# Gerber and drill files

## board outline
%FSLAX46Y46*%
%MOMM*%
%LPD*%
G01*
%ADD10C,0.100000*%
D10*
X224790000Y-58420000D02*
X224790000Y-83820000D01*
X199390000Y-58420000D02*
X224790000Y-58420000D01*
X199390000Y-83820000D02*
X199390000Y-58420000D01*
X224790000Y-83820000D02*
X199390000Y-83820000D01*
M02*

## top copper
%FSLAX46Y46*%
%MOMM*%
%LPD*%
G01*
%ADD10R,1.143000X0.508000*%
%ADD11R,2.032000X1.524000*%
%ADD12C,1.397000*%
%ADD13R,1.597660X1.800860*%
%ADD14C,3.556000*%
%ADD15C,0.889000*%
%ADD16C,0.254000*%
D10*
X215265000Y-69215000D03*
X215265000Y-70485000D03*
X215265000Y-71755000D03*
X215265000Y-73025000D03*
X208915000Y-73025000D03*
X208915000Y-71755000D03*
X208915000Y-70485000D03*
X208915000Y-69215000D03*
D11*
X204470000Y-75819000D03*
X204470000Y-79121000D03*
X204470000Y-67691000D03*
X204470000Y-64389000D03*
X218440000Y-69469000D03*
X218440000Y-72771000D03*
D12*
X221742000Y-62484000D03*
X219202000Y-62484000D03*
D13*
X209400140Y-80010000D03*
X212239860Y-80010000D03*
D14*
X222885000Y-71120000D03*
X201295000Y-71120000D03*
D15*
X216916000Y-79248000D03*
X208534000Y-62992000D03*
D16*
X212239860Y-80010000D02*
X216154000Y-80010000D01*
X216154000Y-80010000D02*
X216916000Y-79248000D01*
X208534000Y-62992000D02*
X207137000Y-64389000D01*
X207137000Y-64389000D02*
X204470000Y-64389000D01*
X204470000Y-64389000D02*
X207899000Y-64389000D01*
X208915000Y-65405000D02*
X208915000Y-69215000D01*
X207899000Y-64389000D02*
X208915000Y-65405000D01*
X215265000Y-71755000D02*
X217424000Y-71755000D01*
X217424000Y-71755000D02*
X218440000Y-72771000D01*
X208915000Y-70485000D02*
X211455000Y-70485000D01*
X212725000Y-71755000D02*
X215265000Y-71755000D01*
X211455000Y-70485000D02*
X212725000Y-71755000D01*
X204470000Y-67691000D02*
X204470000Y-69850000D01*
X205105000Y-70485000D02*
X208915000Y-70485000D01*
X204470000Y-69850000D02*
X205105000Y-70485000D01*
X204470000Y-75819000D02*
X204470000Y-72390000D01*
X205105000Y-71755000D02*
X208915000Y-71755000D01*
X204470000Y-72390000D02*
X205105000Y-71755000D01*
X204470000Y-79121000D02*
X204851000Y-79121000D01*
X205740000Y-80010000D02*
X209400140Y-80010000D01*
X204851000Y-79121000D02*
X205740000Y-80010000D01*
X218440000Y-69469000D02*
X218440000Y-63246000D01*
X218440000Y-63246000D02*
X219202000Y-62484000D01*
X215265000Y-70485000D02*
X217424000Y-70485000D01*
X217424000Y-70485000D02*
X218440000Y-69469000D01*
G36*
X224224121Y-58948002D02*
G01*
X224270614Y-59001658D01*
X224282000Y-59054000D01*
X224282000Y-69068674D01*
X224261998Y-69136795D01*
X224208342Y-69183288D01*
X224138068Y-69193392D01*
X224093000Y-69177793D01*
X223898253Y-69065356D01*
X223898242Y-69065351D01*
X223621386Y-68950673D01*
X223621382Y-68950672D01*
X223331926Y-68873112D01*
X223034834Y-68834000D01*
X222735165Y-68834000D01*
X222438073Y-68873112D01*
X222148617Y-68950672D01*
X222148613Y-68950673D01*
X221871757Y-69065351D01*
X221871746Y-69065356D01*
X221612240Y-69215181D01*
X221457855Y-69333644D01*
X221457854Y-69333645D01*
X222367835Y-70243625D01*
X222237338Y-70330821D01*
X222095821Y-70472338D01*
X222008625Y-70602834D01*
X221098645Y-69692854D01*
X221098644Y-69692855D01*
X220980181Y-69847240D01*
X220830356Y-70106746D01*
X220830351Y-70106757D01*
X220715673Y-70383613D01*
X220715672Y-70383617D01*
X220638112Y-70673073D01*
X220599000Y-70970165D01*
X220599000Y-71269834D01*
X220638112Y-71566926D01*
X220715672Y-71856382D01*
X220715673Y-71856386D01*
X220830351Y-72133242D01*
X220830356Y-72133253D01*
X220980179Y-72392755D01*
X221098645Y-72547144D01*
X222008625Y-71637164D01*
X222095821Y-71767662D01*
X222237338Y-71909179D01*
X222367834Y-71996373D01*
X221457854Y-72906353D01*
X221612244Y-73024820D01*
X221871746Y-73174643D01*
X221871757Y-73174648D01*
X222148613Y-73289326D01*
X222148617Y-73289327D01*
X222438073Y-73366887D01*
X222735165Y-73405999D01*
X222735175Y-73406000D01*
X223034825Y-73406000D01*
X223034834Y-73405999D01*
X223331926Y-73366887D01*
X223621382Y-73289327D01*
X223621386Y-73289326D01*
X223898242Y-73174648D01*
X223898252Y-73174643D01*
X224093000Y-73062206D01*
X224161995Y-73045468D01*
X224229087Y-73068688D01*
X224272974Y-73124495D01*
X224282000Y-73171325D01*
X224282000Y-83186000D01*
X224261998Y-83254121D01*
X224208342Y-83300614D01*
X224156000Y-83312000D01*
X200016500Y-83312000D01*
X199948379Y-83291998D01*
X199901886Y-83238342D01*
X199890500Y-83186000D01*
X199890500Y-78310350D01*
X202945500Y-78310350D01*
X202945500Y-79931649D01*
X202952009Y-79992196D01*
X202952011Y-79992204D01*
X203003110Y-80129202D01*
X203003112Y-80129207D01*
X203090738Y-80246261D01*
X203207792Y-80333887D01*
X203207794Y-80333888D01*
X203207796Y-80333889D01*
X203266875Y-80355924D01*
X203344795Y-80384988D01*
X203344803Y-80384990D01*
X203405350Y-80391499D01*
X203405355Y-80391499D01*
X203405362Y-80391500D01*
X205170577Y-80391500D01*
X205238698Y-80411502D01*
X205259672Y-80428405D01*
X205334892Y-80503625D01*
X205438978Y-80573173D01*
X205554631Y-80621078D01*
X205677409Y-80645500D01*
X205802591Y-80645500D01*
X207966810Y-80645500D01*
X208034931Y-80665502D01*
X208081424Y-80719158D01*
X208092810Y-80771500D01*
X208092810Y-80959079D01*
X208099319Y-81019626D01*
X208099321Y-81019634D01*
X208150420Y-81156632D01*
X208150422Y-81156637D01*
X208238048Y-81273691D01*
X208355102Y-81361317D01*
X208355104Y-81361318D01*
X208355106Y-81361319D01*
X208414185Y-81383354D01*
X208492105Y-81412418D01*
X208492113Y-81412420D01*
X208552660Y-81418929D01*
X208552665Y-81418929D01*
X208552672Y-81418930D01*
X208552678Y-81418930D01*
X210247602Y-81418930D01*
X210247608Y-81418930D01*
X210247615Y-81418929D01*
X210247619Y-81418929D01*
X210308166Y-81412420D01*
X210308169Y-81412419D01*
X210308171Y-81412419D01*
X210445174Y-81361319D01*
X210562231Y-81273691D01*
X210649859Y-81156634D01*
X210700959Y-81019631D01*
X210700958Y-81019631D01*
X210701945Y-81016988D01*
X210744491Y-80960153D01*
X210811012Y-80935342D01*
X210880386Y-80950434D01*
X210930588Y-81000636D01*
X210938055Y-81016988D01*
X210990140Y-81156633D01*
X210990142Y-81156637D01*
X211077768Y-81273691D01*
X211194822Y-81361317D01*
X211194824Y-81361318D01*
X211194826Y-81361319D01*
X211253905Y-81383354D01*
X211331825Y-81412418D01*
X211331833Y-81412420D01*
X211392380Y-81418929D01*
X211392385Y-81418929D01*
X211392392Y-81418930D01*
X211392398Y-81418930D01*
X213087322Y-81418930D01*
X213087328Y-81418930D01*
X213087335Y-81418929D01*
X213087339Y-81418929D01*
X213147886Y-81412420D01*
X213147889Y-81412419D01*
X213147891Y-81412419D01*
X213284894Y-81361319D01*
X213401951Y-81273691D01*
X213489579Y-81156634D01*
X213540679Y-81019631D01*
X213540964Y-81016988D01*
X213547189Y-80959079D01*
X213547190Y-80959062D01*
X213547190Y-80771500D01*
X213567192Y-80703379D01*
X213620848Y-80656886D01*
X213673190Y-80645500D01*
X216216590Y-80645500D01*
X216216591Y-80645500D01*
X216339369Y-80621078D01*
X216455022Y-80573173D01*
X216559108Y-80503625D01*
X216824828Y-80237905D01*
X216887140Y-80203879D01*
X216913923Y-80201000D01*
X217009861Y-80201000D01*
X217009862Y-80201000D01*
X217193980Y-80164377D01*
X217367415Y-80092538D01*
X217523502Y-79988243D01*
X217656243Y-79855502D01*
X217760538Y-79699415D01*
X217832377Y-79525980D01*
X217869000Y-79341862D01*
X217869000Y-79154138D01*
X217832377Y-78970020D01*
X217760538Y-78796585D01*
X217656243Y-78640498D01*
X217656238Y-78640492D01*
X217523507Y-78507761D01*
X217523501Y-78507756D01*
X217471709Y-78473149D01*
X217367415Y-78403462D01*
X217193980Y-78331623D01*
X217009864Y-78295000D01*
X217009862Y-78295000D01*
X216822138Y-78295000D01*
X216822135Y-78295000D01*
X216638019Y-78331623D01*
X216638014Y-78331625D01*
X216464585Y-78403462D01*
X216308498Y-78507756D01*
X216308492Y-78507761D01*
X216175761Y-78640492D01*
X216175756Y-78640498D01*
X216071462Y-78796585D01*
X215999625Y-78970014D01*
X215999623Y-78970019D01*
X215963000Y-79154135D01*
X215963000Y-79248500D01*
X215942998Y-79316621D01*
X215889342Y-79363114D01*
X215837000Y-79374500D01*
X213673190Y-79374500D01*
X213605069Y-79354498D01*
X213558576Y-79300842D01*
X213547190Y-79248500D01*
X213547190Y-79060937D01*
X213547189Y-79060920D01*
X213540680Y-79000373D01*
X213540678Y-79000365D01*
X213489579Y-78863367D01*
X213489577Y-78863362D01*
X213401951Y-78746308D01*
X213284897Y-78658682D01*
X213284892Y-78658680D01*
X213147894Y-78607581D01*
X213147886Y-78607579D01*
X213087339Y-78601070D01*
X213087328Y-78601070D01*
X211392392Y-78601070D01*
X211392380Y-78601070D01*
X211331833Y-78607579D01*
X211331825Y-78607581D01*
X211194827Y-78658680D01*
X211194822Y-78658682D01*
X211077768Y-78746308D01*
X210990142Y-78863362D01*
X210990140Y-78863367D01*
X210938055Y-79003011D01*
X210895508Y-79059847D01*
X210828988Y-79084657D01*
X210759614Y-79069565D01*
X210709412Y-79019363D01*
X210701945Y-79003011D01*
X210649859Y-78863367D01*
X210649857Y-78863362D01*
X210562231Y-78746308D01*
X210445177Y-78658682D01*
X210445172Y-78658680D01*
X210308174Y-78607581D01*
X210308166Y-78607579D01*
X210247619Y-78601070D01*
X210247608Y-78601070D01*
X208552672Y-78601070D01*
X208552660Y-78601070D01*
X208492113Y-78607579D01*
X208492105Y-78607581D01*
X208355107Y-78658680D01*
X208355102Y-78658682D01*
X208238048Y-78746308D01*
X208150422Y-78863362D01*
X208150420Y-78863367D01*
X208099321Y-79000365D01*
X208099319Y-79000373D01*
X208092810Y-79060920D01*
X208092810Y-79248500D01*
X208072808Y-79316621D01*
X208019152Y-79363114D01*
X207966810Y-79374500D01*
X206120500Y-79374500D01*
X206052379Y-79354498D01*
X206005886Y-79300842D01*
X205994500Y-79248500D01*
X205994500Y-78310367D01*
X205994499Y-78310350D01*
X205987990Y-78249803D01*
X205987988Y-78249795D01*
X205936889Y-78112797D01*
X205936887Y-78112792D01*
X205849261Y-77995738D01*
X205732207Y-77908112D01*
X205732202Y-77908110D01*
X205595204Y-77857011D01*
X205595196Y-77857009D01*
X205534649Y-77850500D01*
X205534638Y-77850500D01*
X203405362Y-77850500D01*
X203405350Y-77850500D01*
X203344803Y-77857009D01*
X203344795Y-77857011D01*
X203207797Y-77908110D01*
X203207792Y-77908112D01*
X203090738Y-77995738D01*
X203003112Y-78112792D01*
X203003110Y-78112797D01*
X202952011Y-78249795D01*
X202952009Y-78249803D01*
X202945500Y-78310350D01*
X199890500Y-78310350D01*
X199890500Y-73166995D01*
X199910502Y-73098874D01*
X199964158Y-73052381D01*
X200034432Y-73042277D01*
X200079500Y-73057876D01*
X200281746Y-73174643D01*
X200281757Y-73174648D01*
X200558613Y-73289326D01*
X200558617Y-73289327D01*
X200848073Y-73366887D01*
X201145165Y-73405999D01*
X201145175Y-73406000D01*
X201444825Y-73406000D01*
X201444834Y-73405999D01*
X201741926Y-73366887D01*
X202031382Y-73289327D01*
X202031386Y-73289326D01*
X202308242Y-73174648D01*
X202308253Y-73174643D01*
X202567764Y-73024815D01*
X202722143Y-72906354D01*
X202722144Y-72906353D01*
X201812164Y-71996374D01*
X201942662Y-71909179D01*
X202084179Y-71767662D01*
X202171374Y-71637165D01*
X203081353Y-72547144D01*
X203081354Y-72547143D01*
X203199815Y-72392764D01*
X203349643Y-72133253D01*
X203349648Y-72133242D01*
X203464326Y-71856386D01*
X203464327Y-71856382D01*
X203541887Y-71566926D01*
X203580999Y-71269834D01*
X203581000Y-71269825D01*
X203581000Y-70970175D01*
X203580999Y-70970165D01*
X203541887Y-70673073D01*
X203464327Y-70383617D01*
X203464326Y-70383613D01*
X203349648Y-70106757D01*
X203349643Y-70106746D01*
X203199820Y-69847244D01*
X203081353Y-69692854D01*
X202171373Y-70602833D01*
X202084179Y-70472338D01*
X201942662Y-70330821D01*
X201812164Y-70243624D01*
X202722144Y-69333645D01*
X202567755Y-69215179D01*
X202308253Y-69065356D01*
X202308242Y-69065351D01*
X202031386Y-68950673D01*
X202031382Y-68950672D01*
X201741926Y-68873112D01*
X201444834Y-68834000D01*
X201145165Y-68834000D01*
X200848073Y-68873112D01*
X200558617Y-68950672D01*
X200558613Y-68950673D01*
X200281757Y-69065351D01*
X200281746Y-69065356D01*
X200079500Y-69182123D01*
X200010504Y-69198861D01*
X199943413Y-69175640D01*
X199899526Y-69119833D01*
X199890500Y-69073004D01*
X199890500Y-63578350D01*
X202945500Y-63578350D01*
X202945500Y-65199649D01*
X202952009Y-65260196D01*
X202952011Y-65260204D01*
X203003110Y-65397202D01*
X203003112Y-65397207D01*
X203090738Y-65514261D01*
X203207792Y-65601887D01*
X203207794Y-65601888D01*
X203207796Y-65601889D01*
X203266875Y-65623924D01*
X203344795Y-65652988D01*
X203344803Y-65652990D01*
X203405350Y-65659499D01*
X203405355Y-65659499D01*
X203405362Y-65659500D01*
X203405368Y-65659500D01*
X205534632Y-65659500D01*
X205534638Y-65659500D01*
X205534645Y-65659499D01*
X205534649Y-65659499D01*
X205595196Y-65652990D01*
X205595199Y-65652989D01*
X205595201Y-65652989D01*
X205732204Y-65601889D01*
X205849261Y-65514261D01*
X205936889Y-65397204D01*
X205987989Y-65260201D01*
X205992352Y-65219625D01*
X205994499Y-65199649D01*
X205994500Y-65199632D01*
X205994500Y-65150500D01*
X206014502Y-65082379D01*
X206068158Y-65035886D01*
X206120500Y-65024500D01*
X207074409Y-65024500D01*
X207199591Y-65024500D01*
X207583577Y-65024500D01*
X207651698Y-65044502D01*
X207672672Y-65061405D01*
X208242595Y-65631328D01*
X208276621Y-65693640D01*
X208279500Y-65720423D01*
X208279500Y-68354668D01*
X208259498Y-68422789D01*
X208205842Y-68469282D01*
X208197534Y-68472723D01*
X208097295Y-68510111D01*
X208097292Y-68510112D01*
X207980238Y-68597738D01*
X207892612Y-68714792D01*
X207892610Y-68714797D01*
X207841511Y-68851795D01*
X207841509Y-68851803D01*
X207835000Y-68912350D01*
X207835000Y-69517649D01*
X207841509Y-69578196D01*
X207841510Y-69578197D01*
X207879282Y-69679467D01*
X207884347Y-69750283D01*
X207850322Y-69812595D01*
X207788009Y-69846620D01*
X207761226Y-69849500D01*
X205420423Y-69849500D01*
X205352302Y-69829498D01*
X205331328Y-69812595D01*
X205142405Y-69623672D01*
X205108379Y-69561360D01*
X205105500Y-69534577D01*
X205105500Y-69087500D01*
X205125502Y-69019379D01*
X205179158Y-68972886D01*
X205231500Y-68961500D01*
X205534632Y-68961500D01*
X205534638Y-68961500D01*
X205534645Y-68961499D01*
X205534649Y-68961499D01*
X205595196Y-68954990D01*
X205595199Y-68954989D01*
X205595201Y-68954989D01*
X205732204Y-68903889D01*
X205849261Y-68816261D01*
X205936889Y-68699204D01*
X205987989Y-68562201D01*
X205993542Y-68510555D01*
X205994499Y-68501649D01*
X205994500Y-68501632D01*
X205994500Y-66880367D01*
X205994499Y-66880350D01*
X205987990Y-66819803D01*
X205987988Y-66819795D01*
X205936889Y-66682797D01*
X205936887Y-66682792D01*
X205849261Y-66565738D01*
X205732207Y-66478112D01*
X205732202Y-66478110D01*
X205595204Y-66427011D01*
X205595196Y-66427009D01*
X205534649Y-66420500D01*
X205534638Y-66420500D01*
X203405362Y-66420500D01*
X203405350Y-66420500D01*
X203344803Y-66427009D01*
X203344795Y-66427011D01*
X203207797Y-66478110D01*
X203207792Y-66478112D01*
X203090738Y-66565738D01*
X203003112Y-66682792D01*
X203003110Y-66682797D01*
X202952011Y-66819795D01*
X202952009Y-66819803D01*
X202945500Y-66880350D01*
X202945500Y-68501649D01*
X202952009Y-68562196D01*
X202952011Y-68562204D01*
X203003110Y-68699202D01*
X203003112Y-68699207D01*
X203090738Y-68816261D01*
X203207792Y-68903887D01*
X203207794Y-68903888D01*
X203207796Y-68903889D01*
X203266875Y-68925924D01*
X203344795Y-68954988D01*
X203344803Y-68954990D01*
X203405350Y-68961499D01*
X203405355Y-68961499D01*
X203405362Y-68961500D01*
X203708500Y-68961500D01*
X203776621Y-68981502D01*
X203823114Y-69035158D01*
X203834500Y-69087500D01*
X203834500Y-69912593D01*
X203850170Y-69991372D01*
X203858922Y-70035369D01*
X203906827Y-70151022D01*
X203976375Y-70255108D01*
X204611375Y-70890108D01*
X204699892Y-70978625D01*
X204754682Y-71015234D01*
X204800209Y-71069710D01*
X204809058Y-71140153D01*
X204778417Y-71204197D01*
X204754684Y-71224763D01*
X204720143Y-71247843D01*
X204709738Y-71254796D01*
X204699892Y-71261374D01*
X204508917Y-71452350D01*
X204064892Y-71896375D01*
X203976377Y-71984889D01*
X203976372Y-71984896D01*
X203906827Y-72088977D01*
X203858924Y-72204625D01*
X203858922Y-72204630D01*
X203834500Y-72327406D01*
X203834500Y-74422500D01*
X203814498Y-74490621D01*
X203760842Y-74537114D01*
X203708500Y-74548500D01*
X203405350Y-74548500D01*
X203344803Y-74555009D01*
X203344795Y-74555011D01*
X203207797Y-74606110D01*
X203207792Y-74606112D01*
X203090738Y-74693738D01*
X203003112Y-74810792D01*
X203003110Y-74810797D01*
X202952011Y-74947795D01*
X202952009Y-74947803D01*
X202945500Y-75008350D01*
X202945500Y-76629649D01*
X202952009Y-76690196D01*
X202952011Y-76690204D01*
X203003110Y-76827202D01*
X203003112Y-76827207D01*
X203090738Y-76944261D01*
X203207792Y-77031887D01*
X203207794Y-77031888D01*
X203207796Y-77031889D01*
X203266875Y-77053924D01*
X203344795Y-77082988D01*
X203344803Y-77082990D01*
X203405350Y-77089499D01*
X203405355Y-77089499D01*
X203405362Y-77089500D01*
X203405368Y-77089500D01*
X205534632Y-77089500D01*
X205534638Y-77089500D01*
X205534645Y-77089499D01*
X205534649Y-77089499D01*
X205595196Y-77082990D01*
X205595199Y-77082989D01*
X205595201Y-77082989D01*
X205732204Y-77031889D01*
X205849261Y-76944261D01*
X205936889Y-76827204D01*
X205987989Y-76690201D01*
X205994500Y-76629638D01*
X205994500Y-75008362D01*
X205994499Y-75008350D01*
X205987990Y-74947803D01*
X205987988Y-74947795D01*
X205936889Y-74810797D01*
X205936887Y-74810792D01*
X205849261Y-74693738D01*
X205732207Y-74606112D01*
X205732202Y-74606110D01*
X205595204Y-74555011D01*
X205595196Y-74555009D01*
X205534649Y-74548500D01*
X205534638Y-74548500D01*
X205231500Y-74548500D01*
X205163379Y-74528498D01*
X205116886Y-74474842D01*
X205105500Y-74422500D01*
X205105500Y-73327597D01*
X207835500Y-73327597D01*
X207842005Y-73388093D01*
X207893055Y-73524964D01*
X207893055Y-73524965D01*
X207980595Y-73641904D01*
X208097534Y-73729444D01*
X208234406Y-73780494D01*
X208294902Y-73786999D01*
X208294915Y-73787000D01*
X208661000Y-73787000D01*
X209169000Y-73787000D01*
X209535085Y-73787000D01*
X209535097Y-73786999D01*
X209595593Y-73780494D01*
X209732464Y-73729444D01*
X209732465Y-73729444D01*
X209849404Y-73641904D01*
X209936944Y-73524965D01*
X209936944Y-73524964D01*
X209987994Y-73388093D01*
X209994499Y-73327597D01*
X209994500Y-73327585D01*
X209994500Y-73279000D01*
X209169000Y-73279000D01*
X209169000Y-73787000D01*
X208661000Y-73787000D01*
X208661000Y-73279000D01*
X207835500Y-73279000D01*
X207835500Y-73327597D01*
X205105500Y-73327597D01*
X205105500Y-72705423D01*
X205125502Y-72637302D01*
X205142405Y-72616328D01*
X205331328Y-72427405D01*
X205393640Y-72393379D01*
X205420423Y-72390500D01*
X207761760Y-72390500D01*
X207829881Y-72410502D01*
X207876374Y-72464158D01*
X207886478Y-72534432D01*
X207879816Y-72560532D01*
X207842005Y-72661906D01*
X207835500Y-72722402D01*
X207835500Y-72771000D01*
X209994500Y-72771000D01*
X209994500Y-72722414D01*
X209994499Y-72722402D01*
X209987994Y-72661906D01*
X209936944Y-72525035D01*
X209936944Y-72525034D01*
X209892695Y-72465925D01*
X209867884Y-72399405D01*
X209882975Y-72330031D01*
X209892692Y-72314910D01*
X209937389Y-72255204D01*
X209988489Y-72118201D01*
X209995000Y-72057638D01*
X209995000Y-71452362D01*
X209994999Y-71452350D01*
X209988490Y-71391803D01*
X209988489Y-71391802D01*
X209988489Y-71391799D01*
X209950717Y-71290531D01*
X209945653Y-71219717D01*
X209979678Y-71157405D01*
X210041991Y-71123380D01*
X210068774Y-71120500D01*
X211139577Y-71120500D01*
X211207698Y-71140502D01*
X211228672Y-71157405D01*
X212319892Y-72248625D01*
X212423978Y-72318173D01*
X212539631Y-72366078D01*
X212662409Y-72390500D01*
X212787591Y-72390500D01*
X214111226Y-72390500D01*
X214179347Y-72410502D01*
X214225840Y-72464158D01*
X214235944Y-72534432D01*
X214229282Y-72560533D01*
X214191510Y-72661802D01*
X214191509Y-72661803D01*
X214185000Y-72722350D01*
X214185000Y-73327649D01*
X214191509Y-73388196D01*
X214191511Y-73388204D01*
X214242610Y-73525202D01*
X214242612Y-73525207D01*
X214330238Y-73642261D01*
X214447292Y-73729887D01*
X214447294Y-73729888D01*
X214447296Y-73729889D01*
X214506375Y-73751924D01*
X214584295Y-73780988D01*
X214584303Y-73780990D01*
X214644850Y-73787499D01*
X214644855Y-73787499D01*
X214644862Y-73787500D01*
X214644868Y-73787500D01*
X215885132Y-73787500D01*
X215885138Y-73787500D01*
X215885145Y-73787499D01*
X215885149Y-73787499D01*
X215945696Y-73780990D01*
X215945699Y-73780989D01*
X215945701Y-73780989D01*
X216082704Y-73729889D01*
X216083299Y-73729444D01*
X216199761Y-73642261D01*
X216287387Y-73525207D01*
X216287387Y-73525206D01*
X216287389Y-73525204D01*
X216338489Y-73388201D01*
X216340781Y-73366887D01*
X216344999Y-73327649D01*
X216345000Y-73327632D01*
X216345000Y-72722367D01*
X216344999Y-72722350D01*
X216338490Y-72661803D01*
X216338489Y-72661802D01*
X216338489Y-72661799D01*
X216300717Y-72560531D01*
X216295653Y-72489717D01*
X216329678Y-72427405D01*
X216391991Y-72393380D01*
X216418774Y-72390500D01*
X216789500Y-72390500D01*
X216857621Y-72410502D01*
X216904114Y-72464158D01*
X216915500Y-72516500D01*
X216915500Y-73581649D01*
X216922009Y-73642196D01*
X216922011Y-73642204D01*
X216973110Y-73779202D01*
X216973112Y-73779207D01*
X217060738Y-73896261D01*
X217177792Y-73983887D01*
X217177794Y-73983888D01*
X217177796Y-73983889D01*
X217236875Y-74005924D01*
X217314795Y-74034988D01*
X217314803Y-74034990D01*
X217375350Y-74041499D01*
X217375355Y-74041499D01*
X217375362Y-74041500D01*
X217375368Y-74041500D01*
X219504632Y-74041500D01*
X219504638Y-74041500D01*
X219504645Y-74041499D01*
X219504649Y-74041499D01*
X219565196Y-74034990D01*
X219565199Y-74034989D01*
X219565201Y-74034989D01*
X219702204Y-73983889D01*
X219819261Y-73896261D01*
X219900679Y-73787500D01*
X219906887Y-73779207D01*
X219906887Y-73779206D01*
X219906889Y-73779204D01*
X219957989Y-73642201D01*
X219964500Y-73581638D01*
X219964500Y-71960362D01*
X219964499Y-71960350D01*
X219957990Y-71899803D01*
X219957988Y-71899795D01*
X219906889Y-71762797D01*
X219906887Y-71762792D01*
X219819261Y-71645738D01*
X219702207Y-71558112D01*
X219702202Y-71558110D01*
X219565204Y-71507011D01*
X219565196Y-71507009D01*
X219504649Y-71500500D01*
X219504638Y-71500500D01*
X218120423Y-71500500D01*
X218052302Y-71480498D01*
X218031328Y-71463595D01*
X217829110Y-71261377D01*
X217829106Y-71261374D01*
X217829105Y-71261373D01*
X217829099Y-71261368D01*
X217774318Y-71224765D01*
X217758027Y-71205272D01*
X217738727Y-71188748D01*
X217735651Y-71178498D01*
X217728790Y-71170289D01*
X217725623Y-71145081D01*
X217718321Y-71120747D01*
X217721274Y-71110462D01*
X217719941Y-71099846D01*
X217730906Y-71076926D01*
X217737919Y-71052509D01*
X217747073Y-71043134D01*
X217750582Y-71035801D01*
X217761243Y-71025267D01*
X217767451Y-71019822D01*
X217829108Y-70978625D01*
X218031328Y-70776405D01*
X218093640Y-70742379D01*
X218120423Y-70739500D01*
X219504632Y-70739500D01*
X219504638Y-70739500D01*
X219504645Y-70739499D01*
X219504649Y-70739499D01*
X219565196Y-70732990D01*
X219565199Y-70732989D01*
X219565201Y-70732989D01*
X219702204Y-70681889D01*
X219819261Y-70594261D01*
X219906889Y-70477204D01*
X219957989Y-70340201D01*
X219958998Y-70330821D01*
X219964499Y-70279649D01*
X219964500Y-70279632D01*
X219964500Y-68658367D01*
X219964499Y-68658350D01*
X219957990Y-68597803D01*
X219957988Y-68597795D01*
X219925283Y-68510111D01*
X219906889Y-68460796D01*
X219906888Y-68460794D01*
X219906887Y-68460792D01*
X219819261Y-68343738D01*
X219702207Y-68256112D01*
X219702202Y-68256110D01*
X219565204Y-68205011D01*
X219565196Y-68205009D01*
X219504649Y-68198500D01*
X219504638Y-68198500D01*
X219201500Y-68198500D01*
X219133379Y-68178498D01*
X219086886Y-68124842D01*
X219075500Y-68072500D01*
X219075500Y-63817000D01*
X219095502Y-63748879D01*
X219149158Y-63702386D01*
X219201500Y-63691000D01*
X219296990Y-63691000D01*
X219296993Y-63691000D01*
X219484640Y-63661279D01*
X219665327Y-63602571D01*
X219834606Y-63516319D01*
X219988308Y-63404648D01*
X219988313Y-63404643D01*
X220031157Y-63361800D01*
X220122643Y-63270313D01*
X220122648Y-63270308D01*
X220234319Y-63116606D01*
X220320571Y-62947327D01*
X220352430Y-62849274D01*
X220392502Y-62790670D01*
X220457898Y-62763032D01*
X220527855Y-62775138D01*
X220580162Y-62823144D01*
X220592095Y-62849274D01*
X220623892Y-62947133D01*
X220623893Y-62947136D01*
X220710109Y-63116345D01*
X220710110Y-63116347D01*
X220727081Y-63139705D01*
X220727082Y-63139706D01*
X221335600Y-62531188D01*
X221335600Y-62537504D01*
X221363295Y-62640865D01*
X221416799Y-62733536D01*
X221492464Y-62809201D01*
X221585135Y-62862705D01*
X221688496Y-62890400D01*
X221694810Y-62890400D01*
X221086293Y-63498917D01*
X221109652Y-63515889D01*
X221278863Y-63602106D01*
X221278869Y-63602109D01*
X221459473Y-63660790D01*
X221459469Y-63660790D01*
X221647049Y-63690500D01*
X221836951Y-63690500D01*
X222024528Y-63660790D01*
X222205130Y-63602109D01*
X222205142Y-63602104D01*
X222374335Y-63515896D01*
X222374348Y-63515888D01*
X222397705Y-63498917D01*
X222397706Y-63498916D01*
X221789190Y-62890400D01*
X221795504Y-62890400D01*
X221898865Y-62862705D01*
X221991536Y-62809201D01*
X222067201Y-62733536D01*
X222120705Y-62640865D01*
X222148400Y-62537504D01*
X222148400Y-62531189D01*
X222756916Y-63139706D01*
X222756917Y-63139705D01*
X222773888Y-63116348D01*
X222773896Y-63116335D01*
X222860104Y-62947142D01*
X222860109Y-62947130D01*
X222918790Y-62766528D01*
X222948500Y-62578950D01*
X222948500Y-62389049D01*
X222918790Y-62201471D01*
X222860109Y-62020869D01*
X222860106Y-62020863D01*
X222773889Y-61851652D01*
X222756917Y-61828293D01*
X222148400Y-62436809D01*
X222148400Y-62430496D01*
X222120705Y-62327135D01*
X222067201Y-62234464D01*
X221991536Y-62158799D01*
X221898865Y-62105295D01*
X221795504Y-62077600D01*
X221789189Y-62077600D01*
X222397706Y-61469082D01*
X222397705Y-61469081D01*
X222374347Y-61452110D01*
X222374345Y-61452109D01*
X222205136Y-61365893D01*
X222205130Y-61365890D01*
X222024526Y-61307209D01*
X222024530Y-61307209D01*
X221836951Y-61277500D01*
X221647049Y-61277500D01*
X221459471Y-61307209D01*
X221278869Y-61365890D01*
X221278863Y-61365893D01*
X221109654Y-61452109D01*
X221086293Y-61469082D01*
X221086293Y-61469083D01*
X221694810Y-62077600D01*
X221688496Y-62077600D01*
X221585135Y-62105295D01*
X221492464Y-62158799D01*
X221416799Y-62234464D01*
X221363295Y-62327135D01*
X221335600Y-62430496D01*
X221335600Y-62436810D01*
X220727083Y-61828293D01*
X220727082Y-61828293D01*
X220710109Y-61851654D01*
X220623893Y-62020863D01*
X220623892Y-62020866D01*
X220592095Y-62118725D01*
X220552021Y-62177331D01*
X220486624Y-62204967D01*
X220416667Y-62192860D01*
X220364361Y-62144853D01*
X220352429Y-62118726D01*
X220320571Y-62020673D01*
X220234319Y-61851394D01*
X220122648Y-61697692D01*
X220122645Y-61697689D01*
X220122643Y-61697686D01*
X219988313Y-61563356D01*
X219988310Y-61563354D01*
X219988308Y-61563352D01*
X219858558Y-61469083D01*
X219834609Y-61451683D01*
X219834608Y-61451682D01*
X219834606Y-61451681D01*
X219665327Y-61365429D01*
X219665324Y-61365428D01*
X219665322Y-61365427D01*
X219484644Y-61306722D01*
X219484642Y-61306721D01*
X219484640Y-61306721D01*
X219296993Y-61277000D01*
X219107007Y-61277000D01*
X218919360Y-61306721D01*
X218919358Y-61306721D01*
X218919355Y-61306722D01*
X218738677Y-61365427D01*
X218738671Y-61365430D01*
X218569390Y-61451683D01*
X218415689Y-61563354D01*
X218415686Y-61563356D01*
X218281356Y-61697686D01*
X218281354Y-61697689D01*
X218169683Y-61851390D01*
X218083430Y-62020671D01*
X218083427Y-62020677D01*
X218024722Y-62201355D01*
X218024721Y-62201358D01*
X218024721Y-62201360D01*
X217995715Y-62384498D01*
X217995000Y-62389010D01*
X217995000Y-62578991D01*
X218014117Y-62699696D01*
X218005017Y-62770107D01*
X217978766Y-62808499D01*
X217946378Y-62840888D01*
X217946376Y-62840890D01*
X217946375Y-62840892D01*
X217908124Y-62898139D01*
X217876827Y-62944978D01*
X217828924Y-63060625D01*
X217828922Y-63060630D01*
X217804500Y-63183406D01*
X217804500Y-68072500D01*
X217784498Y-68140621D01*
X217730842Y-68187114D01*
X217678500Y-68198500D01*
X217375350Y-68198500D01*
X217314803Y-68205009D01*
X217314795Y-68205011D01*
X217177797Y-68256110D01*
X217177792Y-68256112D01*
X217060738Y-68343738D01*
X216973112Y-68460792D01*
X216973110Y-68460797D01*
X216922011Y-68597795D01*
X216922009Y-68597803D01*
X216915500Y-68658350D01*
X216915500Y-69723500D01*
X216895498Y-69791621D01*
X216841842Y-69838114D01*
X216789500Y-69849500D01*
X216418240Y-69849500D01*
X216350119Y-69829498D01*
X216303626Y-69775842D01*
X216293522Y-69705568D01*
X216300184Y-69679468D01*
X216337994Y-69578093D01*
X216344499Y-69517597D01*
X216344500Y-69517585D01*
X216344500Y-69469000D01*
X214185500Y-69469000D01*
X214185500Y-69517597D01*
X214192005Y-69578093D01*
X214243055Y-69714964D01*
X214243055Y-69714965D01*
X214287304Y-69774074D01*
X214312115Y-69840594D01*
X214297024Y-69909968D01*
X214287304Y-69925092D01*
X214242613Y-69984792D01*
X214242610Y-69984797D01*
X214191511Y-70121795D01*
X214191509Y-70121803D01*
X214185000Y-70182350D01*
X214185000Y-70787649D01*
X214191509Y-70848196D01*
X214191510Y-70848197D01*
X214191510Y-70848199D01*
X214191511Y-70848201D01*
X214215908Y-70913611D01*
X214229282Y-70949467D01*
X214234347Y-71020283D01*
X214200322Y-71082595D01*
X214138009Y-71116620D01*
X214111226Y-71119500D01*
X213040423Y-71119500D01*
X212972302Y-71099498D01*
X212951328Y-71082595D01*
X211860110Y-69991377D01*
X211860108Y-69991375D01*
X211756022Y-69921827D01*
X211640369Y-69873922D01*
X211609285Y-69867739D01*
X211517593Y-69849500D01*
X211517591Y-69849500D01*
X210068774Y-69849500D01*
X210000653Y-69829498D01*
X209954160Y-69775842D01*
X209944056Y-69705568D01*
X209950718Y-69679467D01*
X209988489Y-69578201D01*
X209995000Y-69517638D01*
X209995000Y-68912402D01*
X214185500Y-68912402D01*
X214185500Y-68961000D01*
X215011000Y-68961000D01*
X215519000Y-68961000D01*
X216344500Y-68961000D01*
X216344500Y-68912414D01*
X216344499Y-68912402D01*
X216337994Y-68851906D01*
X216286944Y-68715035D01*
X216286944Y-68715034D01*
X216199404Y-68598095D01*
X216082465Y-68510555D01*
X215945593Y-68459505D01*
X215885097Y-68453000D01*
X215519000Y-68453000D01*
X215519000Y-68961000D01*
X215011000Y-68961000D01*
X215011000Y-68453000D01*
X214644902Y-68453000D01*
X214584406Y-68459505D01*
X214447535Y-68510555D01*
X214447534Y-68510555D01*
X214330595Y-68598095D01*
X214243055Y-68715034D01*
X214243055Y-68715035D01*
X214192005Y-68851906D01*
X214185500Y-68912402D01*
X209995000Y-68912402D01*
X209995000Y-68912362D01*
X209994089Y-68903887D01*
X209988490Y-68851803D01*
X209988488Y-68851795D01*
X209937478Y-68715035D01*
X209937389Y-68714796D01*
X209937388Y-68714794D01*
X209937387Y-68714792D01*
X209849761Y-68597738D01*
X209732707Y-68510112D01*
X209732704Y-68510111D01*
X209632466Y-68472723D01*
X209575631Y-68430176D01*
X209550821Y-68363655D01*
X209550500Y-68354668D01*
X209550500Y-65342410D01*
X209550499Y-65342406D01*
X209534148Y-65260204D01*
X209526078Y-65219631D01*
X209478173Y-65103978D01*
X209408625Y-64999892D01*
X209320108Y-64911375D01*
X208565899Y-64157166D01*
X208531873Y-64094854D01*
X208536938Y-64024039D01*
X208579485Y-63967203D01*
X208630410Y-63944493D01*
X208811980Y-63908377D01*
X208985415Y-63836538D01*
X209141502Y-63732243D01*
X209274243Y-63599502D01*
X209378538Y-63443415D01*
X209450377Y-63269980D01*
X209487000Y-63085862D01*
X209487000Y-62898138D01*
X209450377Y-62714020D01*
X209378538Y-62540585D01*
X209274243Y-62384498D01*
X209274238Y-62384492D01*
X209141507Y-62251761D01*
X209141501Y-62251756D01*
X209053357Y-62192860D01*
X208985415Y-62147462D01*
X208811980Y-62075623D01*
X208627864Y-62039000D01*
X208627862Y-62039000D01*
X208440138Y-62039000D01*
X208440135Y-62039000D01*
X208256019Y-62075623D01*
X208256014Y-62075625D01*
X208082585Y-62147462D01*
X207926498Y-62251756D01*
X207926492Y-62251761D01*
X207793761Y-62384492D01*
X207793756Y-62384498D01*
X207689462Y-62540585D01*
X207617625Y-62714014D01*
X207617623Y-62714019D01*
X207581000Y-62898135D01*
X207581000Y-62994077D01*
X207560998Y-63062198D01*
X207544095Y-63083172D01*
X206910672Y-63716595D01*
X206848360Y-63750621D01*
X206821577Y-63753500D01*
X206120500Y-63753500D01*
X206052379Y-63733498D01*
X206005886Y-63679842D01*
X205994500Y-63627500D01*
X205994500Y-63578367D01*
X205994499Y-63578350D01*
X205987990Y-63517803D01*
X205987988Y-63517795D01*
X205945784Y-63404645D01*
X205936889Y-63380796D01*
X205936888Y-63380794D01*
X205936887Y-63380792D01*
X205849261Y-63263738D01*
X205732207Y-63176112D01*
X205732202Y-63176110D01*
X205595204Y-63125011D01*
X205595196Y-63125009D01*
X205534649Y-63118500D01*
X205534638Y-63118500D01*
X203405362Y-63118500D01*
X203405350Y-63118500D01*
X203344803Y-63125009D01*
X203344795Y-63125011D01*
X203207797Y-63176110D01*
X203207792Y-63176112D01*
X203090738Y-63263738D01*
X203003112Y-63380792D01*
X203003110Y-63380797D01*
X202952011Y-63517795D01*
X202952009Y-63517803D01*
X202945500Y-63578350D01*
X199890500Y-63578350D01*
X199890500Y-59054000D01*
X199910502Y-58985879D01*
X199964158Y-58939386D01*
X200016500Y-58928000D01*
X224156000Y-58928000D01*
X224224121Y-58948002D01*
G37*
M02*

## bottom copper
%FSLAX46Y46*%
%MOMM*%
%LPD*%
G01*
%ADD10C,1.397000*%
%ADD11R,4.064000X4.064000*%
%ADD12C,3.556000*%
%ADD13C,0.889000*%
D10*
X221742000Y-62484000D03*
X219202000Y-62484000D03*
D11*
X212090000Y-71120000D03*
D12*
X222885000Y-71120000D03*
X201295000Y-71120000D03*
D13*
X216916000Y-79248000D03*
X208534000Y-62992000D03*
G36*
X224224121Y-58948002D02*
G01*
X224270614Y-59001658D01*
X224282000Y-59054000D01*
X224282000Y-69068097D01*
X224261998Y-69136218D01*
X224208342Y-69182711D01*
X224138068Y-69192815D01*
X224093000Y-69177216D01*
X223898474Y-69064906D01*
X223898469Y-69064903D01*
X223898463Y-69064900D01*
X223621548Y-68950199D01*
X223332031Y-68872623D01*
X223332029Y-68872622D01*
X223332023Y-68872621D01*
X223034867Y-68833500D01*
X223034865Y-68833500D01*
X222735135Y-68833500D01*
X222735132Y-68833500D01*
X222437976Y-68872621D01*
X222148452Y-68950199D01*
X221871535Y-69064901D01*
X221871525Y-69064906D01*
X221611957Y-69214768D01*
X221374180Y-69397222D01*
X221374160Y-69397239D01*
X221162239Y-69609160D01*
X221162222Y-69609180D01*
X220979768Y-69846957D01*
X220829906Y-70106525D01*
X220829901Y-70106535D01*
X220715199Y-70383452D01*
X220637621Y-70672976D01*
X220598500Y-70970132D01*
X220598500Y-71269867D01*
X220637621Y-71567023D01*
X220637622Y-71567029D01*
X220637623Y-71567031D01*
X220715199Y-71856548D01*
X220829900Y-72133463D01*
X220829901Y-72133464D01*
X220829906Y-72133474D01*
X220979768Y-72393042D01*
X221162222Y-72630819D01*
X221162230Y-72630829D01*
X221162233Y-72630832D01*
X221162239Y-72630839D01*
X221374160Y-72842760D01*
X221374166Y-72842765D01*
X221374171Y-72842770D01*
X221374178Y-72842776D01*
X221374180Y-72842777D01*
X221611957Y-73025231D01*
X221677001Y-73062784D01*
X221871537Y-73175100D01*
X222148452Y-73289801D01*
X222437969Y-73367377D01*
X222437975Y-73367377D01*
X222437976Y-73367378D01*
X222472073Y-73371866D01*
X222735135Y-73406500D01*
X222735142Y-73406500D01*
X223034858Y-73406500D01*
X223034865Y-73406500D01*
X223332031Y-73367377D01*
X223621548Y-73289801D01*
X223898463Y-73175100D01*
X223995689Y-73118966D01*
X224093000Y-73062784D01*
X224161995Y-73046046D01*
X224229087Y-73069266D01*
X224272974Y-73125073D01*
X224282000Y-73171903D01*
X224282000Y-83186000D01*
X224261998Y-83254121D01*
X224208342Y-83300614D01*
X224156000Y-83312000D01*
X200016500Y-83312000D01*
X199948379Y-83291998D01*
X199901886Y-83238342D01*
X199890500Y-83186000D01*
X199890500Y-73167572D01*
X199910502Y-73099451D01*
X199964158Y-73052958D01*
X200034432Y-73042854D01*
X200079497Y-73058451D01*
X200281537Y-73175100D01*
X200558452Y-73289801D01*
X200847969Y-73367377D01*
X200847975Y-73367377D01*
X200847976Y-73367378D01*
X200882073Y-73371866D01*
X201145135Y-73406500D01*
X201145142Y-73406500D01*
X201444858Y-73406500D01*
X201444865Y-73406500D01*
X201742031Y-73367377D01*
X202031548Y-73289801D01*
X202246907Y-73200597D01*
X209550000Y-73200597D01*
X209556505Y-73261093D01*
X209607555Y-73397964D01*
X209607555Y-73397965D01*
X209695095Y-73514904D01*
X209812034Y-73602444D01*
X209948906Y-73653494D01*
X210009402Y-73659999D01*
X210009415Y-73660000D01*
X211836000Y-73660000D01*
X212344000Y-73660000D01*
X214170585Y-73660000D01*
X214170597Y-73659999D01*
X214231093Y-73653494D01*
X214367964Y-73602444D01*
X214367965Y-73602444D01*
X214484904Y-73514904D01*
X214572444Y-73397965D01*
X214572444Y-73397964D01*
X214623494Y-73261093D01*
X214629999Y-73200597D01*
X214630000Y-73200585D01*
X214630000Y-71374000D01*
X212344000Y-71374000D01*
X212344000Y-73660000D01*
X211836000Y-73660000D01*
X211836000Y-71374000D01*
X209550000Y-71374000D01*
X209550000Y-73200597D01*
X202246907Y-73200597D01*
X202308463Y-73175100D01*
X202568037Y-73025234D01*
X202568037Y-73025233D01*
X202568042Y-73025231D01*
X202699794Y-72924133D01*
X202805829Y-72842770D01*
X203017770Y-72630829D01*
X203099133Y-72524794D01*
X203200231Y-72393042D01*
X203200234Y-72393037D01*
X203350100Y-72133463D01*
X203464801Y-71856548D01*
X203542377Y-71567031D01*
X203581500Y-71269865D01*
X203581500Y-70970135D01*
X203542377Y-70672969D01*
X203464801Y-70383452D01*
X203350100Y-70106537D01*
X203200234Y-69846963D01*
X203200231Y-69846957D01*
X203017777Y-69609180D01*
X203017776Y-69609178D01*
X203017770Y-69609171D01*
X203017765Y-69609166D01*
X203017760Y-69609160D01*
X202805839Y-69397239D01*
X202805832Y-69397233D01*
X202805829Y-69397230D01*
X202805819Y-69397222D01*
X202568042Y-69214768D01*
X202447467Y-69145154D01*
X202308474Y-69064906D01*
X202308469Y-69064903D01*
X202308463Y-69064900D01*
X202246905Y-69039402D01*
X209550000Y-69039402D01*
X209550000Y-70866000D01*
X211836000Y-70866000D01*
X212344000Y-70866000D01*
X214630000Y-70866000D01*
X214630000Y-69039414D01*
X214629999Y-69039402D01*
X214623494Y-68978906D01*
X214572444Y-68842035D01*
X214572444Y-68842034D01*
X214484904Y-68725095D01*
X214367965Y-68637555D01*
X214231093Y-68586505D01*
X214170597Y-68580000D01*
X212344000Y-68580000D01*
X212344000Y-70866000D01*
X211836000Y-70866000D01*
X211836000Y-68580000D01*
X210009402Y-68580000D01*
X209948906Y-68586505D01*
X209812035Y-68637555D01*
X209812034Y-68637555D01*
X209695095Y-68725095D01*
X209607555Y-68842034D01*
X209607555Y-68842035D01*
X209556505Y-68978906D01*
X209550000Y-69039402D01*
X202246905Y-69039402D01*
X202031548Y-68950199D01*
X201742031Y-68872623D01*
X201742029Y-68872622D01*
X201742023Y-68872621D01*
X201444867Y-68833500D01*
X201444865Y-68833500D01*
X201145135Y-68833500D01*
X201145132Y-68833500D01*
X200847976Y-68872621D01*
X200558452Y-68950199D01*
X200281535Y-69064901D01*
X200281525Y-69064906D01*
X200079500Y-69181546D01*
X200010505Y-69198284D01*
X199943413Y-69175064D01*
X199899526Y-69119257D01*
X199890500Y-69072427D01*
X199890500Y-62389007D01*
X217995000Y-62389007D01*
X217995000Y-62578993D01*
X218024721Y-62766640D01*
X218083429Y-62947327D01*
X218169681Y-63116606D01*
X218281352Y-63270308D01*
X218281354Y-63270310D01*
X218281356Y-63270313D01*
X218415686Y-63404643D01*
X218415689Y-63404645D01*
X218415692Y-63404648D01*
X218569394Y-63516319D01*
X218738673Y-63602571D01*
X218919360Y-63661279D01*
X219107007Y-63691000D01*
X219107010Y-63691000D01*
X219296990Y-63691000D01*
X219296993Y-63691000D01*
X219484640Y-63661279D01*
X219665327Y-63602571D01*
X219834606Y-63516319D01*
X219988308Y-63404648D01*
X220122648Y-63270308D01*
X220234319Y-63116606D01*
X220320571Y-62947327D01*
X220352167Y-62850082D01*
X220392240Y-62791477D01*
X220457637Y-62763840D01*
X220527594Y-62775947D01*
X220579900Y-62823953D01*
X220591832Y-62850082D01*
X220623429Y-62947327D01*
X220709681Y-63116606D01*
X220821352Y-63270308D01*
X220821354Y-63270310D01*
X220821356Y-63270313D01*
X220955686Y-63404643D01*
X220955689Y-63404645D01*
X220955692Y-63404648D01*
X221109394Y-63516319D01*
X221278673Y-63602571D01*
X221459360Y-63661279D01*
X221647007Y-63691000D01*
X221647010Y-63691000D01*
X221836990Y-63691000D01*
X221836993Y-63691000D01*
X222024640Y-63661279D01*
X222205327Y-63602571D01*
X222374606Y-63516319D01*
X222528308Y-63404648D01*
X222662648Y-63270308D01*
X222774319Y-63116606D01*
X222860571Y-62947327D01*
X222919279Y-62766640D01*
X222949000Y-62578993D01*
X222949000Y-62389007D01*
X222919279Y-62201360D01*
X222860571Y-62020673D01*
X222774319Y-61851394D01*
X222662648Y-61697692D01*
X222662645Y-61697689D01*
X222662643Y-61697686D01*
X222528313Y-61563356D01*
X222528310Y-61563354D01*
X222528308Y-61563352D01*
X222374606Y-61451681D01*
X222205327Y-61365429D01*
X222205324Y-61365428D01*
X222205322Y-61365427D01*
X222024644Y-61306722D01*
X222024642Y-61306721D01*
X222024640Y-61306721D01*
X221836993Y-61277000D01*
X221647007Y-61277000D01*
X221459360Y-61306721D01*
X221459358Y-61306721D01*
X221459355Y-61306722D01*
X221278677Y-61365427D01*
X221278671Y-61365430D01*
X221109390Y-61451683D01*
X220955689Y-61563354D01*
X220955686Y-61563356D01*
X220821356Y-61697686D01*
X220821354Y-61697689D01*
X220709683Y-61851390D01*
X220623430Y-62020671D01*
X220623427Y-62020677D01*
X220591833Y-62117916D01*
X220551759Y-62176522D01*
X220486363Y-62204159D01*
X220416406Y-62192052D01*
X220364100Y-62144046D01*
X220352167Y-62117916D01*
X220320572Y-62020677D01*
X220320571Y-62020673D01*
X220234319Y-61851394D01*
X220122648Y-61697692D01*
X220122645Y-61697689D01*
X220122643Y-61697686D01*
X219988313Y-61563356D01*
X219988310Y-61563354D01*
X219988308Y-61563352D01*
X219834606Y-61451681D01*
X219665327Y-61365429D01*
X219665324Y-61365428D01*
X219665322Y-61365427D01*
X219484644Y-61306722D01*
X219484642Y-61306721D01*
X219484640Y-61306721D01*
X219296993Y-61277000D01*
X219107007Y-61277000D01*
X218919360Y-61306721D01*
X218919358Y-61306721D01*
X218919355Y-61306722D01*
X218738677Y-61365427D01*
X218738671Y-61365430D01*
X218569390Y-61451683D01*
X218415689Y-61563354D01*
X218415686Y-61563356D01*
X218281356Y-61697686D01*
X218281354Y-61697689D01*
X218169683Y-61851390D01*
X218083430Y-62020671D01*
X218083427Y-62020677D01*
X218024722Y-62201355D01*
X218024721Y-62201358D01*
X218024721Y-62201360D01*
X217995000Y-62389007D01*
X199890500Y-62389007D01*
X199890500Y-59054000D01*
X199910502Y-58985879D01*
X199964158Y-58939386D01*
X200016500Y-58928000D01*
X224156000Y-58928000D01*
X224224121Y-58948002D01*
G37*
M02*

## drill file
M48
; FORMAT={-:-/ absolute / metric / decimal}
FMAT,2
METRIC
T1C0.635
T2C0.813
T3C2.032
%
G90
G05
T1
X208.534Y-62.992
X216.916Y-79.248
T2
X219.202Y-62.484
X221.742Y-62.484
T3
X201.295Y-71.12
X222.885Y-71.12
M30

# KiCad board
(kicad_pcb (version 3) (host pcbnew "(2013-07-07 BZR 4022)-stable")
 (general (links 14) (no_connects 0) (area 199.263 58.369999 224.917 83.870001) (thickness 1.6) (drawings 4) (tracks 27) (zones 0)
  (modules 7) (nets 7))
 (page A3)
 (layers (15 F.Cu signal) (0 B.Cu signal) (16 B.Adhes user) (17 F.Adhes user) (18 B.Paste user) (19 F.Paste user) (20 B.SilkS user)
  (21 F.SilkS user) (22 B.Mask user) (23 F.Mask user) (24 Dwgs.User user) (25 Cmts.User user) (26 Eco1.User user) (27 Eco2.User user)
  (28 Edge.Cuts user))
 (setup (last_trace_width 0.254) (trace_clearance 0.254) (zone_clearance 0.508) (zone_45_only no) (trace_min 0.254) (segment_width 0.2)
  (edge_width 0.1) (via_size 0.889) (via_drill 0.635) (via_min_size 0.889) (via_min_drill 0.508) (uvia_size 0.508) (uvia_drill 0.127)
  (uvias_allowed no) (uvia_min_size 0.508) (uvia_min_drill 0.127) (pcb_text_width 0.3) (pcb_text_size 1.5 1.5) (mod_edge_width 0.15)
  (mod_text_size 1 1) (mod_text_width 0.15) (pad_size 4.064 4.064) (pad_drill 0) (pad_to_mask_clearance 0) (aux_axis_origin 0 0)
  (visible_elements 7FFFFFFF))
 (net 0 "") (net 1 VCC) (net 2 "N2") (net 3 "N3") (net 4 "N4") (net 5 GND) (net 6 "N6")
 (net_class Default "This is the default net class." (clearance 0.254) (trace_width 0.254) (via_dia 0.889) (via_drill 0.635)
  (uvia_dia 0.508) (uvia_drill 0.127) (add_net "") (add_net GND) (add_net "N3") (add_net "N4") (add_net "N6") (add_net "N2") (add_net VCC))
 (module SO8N (layer F.Cu) (at 212.09 71.12 270)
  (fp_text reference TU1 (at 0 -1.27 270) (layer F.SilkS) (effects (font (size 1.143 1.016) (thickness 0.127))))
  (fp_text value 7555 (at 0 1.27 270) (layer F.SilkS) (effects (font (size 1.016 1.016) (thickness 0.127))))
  (pad 8 smd rect (at -1.905 -3.175 270) (size 0.508 1.143) (layers F.Cu F.Paste F.Mask) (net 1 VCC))
  (pad 7 smd rect (at -0.635 -3.175 270) (size 0.508 1.143) (layers F.Cu F.Paste F.Mask) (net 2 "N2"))
  (pad 6 smd rect (at 0.635 -3.175 270) (size 0.508 1.143) (layers F.Cu F.Paste F.Mask) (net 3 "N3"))
  (pad 5 smd rect (at 1.905 -3.175 270) (size 0.508 1.143) (layers F.Cu F.Paste F.Mask))
  (pad 4 smd rect (at 1.905 3.175 270) (size 0.508 1.143) (layers F.Cu F.Paste F.Mask) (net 1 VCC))
  (pad 3 smd rect (at 0.635 3.175 270) (size 0.508 1.143) (layers F.Cu F.Paste F.Mask) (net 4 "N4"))
  (pad 2 smd rect (at -0.635 3.175 270) (size 0.508 1.143) (layers F.Cu F.Paste F.Mask) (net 3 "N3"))
  (pad 1 smd rect (at -1.905 3.175 270) (size 0.508 1.143) (layers F.Cu F.Paste F.Mask) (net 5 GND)))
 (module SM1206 (layer F.Cu) (at 204.47 77.47 270)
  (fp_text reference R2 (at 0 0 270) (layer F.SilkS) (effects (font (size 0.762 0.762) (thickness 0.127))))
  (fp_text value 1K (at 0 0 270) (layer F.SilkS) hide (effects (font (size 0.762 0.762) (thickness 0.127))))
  (pad 1 smd rect (at -1.651 0 270) (size 1.524 2.032) (layers F.Cu F.Paste F.Mask) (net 4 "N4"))
  (pad 2 smd rect (at 1.651 0 270) (size 1.524 2.032) (layers F.Cu F.Paste F.Mask) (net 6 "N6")))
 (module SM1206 (layer F.Cu) (at 204.47 66.04 90)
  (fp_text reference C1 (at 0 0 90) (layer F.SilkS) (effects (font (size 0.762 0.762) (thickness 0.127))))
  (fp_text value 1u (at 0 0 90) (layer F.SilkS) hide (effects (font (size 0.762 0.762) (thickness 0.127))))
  (pad 1 smd rect (at -1.651 0 90) (size 1.524 2.032) (layers F.Cu F.Paste F.Mask) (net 3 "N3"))
  (pad 2 smd rect (at 1.651 0 90) (size 1.524 2.032) (layers F.Cu F.Paste F.Mask) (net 5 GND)))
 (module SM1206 (layer F.Cu) (at 218.44 71.12 270)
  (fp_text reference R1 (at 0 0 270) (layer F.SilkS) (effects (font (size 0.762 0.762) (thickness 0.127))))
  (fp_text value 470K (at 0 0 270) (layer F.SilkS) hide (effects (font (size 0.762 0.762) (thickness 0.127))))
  (pad 1 smd rect (at -1.651 0 270) (size 1.524 2.032) (layers F.Cu F.Paste F.Mask) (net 2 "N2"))
  (pad 2 smd rect (at 1.651 0 270) (size 1.524 2.032) (layers F.Cu F.Paste F.Mask) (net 3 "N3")))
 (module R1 (layer F.Cu) (at 220.472 62.484 180) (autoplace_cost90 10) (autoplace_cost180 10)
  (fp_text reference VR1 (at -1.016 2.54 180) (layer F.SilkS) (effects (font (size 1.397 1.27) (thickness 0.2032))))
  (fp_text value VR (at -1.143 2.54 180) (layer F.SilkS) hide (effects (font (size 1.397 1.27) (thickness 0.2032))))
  (pad 1 thru_hole circle (at -1.27 0 180) (size 1.397 1.397) (drill 0.8128) (layers *.Cu *.Mask F.SilkS) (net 1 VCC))
  (pad 2 thru_hole circle (at 1.27 0 180) (size 1.397 1.397) (drill 0.8128) (layers *.Cu *.Mask F.SilkS) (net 2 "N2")))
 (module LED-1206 (layer F.Cu) (at 210.82 80.01)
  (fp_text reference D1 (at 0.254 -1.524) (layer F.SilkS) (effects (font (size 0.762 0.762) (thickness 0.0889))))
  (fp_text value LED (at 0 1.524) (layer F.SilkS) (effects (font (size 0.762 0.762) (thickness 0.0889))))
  (pad 1 smd rect (at -1.41986 0) (size 1.59766 1.80086) (layers F.Cu F.Paste F.Mask) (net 6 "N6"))
  (pad 2 smd rect (at 1.41986 0) (size 1.59766 1.80086) (layers F.Cu F.Paste F.Mask) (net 5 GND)))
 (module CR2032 (layer B.Cu) (at 212.09 71.12 180)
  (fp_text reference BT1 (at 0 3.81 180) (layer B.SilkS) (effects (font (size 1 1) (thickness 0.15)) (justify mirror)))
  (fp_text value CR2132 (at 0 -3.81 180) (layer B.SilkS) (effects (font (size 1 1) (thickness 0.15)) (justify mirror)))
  (pad 2 smd rect (at 0 0 180) (size 4.064 4.064) (layers B.Cu B.Paste B.Mask) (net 5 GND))
  (pad 1 thru_hole circle (at -10.795 0 180) (size 3.556 3.556) (drill 2.032) (layers *.Cu *.Mask B.SilkS) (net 1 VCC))
  (pad 1 thru_hole circle (at 10.795 0 180) (size 3.556 3.556) (drill 2.032) (layers *.Cu *.Mask B.SilkS) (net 1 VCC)))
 (gr_line (start 224.79 58.42) (end 224.79 83.82) (angle 90) (layer Edge.Cuts) (width 0.1))
 (gr_line (start 199.39 58.42) (end 224.79 58.42) (angle 90) (layer Edge.Cuts) (width 0.1))
 (gr_line (start 199.39 83.82) (end 199.39 58.42) (angle 90) (layer Edge.Cuts) (width 0.1))
 (gr_line (start 224.79 83.82) (end 199.39 83.82) (angle 90) (layer Edge.Cuts) (width 0.1))
 (segment (start 212.23986 80.01) (end 216.154 80.01) (width 0.254) (layer F.Cu) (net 5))
 (via (at 216.916 79.248) (size 0.889) (layers F.Cu B.Cu) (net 5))
 (segment (start 216.154 80.01) (end 216.916 79.248) (width 0.254) (layer F.Cu) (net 5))
 (via (at 208.534 62.992) (size 0.889) (layers F.Cu B.Cu) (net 5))
 (segment (start 208.534 62.992) (end 207.137 64.389) (width 0.254) (layer F.Cu) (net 5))
 (segment (start 207.137 64.389) (end 204.47 64.389) (width 0.254) (layer F.Cu) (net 5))
 (segment (start 204.47 64.389) (end 207.899 64.389) (width 0.254) (layer F.Cu) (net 5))
 (segment (start 208.915 65.405) (end 208.915 69.215) (width 0.254) (layer F.Cu) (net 5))
 (segment (start 207.899 64.389) (end 208.915 65.405) (width 0.254) (layer F.Cu) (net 5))
 (segment (start 215.265 71.755) (end 217.424 71.755) (width 0.254) (layer F.Cu) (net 3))
 (segment (start 217.424 71.755) (end 218.44 72.771) (width 0.254) (layer F.Cu) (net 3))
 (segment (start 208.915 70.485) (end 211.455 70.485) (width 0.254) (layer F.Cu) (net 3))
 (segment (start 212.725 71.755) (end 215.265 71.755) (width 0.254) (layer F.Cu) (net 3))
 (segment (start 211.455 70.485) (end 212.725 71.755) (width 0.254) (layer F.Cu) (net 3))
 (segment (start 204.47 67.691) (end 204.47 69.85) (width 0.254) (layer F.Cu) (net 3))
 (segment (start 205.105 70.485) (end 208.915 70.485) (width 0.254) (layer F.Cu) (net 3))
 (segment (start 204.47 69.85) (end 205.105 70.485) (width 0.254) (layer F.Cu) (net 3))
 (segment (start 204.47 75.819) (end 204.47 72.39) (width 0.254) (layer F.Cu) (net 4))
 (segment (start 205.105 71.755) (end 208.915 71.755) (width 0.254) (layer F.Cu) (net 4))
 (segment (start 204.47 72.39) (end 205.105 71.755) (width 0.254) (layer F.Cu) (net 4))
 (segment (start 204.47 79.121) (end 204.851 79.121) (width 0.254) (layer F.Cu) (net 6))
 (segment (start 205.74 80.01) (end 209.40014 80.01) (width 0.254) (layer F.Cu) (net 6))
 (segment (start 204.851 79.121) (end 205.74 80.01) (width 0.254) (layer F.Cu) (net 6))
 (segment (start 218.44 69.469) (end 218.44 63.246) (width 0.254) (layer F.Cu) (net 2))
 (segment (start 218.44 63.246) (end 219.202 62.484) (width 0.254) (layer F.Cu) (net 2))
 (segment (start 215.265 70.485) (end 217.424 70.485) (width 0.254) (layer F.Cu) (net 2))
 (segment (start 217.424 70.485) (end 218.44 69.469) (width 0.254) (layer F.Cu) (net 2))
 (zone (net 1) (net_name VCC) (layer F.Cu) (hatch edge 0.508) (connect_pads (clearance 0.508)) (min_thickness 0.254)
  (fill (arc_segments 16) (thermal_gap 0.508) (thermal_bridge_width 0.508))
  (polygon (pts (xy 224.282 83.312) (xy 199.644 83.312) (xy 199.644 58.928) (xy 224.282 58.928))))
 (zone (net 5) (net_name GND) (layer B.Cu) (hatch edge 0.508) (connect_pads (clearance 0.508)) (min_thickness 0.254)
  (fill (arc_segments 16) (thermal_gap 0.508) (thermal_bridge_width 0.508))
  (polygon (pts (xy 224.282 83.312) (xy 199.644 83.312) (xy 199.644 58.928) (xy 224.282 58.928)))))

